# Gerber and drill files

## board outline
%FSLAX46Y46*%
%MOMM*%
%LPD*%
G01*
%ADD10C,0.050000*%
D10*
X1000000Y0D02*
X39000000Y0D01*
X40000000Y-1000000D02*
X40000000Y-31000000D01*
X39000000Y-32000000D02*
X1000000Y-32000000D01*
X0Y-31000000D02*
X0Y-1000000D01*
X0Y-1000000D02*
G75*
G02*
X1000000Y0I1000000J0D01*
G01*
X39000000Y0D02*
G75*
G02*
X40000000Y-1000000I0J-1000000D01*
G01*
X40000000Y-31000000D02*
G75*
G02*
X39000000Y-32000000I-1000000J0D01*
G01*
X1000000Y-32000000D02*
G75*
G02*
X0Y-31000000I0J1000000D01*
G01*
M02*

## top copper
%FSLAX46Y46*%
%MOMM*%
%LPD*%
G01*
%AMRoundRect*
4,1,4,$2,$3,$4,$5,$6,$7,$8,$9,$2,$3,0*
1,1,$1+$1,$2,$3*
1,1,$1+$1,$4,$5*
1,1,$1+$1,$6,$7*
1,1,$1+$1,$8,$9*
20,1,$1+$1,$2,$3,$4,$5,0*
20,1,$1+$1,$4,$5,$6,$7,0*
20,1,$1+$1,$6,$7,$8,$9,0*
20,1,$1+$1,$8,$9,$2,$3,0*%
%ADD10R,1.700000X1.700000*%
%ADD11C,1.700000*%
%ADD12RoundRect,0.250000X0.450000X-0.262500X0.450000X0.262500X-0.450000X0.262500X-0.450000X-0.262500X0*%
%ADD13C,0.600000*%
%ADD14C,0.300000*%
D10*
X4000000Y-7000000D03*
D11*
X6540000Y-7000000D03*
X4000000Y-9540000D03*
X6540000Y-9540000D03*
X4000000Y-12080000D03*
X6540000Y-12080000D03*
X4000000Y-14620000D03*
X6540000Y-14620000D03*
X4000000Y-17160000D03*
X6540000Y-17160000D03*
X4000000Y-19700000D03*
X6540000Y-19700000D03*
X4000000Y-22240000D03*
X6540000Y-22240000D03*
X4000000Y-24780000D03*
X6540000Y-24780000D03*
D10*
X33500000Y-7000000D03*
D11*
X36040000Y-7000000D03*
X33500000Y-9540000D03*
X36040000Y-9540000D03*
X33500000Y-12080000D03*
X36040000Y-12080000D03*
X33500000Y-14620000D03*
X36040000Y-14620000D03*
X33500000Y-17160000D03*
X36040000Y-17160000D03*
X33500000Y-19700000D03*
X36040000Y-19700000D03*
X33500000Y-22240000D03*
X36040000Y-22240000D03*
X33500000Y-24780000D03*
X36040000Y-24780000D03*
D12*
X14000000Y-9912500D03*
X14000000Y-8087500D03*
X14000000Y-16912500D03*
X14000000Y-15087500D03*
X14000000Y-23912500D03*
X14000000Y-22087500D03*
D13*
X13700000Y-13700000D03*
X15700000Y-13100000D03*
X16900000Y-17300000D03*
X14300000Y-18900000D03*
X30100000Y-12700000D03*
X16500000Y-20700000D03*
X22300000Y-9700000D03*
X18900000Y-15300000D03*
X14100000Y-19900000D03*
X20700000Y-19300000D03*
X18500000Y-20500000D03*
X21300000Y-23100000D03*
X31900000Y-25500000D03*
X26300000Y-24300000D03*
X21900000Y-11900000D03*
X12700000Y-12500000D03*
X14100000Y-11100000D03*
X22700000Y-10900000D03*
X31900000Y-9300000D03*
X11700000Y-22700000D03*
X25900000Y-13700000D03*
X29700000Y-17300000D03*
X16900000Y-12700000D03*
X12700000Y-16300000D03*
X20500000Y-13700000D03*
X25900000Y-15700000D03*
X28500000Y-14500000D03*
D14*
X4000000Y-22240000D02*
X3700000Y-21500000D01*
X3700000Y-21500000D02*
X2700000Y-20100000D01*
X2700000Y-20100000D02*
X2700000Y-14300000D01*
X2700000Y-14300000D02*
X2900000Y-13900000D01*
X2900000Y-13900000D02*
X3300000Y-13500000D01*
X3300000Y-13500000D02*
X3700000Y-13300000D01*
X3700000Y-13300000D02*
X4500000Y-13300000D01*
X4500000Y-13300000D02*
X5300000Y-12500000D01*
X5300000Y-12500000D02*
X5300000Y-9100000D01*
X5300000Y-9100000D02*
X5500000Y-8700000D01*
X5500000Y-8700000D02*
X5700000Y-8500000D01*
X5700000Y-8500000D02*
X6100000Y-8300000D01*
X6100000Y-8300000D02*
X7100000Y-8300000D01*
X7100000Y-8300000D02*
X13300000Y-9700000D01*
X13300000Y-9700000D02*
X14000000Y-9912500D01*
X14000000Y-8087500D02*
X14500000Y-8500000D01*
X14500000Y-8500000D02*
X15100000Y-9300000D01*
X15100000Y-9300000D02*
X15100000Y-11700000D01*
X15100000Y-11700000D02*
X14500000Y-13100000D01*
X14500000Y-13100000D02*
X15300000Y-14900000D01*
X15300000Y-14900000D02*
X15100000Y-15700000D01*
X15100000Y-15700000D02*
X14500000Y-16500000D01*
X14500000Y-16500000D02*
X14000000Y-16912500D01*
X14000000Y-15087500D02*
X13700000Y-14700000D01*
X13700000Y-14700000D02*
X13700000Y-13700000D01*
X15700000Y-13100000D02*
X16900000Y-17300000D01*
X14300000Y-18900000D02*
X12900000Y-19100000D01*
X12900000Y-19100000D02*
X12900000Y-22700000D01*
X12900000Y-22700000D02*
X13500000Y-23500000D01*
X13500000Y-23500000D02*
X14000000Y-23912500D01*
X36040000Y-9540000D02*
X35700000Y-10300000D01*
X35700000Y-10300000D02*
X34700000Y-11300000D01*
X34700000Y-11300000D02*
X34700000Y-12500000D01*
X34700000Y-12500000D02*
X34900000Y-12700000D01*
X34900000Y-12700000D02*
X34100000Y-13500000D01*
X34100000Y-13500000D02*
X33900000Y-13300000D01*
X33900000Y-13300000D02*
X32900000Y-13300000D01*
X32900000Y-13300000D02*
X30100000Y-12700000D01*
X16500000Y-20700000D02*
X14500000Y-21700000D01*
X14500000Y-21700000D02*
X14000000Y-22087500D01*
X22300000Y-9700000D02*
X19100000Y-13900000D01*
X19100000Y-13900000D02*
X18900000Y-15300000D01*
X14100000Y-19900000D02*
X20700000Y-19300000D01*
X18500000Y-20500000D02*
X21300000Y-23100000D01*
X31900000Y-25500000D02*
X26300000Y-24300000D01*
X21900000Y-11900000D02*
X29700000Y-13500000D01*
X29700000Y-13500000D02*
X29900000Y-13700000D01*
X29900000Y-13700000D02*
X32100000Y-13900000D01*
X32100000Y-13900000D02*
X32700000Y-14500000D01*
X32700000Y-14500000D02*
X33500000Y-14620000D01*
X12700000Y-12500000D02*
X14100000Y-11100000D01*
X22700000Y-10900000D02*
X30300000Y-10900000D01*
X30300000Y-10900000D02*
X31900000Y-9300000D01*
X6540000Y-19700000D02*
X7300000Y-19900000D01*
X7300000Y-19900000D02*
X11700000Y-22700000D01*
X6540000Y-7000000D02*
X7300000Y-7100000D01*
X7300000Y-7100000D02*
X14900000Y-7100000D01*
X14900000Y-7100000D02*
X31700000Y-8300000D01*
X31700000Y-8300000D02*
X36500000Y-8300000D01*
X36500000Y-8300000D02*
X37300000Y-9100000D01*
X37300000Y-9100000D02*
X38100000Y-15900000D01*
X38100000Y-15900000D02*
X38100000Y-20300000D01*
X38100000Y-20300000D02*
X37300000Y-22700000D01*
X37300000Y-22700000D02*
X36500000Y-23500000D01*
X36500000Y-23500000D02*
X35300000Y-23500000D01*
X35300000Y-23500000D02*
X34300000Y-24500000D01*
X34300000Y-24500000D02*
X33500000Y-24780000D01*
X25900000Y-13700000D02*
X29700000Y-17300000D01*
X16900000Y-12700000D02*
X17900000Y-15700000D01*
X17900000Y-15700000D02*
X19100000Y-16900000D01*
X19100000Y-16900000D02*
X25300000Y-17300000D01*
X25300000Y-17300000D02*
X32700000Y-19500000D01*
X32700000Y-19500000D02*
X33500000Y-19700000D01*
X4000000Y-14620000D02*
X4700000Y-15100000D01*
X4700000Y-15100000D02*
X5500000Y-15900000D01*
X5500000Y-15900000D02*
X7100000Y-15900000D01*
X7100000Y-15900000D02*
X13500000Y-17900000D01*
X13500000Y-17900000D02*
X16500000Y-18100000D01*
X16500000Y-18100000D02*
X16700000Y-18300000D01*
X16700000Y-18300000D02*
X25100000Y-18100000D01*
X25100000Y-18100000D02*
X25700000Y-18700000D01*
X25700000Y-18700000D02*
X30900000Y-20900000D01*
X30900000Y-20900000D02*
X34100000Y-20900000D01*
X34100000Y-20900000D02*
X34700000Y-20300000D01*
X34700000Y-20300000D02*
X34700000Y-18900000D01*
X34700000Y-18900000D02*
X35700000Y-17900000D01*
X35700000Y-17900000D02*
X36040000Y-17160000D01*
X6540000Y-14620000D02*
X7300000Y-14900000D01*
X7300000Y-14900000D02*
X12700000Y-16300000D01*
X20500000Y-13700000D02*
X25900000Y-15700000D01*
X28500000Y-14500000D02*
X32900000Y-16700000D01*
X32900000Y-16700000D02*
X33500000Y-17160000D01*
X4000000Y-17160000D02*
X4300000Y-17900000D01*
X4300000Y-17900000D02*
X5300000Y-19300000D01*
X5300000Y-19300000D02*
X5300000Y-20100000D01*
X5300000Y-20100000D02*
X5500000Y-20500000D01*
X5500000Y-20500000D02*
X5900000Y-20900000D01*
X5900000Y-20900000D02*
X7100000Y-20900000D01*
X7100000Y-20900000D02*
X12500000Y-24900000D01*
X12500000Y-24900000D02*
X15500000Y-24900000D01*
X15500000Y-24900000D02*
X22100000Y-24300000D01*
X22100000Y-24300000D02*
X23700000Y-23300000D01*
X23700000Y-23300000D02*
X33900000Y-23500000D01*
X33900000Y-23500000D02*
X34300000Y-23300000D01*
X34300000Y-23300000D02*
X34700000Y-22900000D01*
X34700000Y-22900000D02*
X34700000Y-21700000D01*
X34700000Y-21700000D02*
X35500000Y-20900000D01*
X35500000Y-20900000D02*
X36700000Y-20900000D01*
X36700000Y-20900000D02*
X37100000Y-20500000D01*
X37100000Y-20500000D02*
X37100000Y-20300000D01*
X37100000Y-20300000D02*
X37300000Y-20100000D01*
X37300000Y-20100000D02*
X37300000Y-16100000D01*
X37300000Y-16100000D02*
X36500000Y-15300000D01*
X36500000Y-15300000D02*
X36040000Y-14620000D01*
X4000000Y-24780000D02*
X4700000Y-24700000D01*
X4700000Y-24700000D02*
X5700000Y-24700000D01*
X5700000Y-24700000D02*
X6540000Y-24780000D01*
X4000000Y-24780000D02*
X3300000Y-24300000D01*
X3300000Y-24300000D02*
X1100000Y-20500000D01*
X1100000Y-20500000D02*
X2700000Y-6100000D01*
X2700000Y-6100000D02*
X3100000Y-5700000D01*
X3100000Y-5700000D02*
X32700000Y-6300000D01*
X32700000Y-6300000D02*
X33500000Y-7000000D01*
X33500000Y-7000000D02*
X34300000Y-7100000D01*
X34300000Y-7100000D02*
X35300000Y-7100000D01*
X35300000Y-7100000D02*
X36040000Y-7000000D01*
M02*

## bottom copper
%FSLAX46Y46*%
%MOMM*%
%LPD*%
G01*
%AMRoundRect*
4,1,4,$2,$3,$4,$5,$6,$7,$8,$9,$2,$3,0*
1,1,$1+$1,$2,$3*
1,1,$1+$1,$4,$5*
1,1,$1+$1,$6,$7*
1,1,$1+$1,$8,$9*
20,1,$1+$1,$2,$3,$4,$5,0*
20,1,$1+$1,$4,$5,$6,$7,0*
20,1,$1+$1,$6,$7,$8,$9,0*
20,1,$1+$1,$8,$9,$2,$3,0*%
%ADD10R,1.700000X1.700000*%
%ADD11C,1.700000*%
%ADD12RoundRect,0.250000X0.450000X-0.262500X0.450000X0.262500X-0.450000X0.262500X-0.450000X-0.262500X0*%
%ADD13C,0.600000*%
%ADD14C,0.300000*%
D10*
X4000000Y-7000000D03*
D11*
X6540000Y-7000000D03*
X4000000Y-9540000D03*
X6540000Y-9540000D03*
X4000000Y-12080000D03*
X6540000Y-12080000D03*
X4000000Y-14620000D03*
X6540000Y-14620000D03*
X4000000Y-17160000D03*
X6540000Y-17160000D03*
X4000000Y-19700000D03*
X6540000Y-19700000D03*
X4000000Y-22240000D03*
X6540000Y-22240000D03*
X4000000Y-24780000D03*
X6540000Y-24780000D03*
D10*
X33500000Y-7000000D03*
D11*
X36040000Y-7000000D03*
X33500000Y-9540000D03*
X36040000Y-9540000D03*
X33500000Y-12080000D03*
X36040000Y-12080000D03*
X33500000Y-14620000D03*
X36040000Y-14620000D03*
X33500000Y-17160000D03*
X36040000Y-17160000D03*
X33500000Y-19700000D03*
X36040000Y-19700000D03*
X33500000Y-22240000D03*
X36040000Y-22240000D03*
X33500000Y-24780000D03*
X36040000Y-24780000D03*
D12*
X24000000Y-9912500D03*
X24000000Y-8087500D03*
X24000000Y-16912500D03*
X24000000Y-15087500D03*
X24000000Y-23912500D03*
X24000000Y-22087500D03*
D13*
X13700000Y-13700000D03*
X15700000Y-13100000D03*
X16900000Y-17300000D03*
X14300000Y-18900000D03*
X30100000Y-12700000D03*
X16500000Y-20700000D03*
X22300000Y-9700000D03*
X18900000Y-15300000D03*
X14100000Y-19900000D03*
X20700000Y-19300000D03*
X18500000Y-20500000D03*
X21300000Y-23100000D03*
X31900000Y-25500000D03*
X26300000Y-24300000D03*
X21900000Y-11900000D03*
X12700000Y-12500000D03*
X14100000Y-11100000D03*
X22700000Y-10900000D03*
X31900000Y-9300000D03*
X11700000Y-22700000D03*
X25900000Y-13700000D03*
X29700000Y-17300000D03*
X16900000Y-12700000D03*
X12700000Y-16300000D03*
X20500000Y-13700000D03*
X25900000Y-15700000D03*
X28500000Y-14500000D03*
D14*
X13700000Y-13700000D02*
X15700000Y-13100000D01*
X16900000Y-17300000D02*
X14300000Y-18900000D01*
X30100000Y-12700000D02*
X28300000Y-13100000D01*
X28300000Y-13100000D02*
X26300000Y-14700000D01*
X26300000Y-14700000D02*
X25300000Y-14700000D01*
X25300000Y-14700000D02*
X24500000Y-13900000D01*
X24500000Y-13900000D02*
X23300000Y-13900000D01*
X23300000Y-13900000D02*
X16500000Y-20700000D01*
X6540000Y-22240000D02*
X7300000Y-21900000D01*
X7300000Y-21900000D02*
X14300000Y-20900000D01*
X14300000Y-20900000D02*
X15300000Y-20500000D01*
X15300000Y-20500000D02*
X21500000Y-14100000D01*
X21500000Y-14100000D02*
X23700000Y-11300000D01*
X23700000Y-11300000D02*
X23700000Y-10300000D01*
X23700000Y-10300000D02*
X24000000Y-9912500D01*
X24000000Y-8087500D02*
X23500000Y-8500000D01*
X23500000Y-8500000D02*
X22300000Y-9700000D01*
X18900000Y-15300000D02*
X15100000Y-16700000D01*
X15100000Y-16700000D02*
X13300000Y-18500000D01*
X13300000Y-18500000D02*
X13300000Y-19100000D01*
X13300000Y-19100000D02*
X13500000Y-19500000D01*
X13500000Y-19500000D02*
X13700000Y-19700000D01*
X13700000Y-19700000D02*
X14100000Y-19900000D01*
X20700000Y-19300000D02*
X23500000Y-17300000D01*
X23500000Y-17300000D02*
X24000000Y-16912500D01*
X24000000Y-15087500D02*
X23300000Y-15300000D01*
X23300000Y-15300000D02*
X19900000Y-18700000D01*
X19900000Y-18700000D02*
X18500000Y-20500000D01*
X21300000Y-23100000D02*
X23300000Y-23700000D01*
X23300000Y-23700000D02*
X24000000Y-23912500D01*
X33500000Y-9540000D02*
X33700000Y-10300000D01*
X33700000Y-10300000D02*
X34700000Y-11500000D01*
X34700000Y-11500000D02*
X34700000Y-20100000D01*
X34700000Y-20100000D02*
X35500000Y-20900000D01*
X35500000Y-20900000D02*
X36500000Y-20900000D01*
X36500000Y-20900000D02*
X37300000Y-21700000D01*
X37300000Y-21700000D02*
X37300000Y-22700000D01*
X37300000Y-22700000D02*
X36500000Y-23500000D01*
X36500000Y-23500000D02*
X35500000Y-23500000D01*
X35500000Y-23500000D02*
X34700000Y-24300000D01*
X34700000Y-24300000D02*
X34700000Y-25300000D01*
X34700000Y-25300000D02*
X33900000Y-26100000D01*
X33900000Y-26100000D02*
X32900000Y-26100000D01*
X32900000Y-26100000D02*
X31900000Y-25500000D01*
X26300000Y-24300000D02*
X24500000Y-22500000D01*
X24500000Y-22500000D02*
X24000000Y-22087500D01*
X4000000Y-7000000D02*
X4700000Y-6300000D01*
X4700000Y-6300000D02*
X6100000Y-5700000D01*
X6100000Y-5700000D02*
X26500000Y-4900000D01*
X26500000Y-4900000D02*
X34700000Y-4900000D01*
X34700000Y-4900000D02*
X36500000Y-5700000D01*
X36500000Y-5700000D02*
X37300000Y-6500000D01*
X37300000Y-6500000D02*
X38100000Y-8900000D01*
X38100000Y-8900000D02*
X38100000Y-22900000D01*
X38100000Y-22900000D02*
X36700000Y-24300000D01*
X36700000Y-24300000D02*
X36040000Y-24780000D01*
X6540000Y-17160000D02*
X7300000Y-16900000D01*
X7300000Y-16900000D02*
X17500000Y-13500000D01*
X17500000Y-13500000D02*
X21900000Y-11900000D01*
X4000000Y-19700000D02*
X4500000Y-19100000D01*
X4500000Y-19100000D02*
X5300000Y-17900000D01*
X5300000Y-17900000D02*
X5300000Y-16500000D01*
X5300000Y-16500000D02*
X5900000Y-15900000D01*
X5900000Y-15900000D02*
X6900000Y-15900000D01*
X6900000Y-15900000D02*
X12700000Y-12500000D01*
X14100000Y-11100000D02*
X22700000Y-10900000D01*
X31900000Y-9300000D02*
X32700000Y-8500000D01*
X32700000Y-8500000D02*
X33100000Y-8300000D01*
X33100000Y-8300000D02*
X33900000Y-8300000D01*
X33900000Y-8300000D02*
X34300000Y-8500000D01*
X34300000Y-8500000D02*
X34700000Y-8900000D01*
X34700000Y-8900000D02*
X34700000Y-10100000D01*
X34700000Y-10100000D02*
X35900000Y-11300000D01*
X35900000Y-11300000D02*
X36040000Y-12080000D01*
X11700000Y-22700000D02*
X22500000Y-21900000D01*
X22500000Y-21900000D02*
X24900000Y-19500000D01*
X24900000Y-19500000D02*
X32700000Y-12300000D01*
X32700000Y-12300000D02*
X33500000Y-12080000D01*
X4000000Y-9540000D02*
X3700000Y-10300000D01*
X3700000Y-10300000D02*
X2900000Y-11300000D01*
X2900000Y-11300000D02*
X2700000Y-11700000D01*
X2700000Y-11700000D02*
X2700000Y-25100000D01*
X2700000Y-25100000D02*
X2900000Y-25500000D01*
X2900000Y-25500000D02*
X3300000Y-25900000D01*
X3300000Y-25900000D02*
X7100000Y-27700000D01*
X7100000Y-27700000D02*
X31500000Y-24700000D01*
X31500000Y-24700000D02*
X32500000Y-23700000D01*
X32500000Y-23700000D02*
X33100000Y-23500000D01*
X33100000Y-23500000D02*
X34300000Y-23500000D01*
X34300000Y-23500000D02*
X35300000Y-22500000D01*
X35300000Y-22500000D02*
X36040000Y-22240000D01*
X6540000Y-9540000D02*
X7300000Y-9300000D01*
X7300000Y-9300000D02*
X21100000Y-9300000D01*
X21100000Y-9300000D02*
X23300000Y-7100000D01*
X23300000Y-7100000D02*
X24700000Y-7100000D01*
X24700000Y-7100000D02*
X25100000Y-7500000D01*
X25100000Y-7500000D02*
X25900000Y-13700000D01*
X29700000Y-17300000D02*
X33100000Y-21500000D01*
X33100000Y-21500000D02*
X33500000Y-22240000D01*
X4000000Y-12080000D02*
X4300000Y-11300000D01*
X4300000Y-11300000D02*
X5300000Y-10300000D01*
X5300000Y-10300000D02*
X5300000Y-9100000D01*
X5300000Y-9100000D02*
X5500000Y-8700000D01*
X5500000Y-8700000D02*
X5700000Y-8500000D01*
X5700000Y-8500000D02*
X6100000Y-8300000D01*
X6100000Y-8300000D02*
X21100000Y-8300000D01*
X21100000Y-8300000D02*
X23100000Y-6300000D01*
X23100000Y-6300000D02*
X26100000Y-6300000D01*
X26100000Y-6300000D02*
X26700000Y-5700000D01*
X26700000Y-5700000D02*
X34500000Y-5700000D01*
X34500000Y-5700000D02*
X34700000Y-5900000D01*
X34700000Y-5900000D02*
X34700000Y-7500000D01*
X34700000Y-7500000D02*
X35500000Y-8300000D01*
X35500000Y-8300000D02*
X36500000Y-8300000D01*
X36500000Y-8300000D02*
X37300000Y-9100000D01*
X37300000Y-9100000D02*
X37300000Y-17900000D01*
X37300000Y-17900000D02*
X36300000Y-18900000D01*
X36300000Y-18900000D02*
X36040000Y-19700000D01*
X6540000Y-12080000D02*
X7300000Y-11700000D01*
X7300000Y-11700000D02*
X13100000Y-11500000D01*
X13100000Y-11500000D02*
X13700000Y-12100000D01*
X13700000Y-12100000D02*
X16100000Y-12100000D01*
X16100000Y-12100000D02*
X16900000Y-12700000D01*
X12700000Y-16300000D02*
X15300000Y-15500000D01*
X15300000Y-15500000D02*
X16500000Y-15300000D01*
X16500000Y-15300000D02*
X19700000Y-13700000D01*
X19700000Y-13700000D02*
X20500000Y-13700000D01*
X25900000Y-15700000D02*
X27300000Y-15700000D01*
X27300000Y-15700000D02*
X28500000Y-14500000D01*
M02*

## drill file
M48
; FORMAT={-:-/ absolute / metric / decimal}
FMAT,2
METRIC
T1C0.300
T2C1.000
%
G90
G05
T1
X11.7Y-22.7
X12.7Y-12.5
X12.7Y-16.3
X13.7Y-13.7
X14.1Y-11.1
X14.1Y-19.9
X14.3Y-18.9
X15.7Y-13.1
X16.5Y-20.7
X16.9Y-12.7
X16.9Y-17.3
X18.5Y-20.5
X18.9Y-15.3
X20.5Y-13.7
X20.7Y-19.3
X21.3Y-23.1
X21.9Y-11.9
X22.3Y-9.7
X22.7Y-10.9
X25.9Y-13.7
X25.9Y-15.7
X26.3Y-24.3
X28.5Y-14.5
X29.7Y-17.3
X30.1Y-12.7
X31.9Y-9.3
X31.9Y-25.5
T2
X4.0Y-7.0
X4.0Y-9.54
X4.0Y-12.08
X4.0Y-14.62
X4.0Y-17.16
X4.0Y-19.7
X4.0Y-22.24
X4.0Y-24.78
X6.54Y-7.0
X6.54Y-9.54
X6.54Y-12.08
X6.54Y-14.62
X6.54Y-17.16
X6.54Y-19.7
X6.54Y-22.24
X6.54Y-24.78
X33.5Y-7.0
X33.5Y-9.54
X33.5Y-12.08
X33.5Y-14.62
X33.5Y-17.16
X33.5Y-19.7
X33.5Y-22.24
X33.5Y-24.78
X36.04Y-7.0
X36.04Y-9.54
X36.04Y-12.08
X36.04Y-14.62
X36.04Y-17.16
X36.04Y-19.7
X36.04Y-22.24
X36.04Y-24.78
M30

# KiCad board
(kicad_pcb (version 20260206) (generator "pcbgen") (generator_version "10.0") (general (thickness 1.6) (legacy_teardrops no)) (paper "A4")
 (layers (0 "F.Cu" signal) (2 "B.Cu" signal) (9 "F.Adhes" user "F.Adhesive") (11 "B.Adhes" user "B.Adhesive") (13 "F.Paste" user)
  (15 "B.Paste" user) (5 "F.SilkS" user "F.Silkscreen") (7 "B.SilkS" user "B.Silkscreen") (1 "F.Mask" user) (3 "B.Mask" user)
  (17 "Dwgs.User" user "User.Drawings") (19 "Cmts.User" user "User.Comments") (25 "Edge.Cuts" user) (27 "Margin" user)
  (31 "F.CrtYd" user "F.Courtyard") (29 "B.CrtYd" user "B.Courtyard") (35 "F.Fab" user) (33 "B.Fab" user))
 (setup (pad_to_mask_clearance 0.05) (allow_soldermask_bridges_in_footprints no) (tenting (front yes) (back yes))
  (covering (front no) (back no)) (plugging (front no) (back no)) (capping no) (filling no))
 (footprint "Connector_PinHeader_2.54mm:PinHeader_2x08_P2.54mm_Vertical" (layer "F.Cu") (at 4 7)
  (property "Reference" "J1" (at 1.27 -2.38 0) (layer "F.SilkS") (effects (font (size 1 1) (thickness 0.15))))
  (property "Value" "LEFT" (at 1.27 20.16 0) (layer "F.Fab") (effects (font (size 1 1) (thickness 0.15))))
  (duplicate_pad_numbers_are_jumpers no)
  (pad "1" thru_hole rect (at 0 0) (size 1.7 1.7) (drill 1) (layers "*.Cu" "*.Mask") (remove_unused_layers no) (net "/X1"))
  (pad "2" thru_hole circle (at 2.54 0) (size 1.7 1.7) (drill 1) (layers "*.Cu" "*.Mask") (remove_unused_layers no) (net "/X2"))
  (pad "3" thru_hole circle (at 0 2.54) (size 1.7 1.7) (drill 1) (layers "*.Cu" "*.Mask") (remove_unused_layers no) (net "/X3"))
  (pad "4" thru_hole circle (at 2.54 2.54) (size 1.7 1.7) (drill 1) (layers "*.Cu" "*.Mask") (remove_unused_layers no) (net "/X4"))
  (pad "5" thru_hole circle (at 0 5.08) (size 1.7 1.7) (drill 1) (layers "*.Cu" "*.Mask") (remove_unused_layers no) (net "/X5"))
  (pad "6" thru_hole circle (at 2.54 5.08) (size 1.7 1.7) (drill 1) (layers "*.Cu" "*.Mask") (remove_unused_layers no) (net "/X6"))
  (pad "7" thru_hole circle (at 0 7.62) (size 1.7 1.7) (drill 1) (layers "*.Cu" "*.Mask") (remove_unused_layers no) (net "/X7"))
  (pad "8" thru_hole circle (at 2.54 7.62) (size 1.7 1.7) (drill 1) (layers "*.Cu" "*.Mask") (remove_unused_layers no) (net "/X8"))
  (pad "9" thru_hole circle (at 0 10.16) (size 1.7 1.7) (drill 1) (layers "*.Cu" "*.Mask") (remove_unused_layers no) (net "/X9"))
  (pad "10" thru_hole circle (at 2.54 10.16) (size 1.7 1.7) (drill 1) (layers "*.Cu" "*.Mask") (remove_unused_layers no) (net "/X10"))
  (pad "11" thru_hole circle (at 0 12.7) (size 1.7 1.7) (drill 1) (layers "*.Cu" "*.Mask") (remove_unused_layers no) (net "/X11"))
  (pad "12" thru_hole circle (at 2.54 12.7) (size 1.7 1.7) (drill 1) (layers "*.Cu" "*.Mask") (remove_unused_layers no) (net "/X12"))
  (pad "13" thru_hole circle (at 0 15.24) (size 1.7 1.7) (drill 1) (layers "*.Cu" "*.Mask") (remove_unused_layers no) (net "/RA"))
  (pad "14" thru_hole circle (at 2.54 15.24) (size 1.7 1.7) (drill 1) (layers "*.Cu" "*.Mask") (remove_unused_layers no) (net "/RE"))
  (pad "15" thru_hole circle (at 0 17.78) (size 1.7 1.7) (drill 1) (layers "*.Cu" "*.Mask") (remove_unused_layers no) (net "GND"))
  (pad "16" thru_hole circle (at 2.54 17.78) (size 1.7 1.7) (drill 1) (layers "*.Cu" "*.Mask") (remove_unused_layers no) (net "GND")))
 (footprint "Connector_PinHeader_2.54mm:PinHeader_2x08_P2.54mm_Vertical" (layer "F.Cu") (at 33.5 7)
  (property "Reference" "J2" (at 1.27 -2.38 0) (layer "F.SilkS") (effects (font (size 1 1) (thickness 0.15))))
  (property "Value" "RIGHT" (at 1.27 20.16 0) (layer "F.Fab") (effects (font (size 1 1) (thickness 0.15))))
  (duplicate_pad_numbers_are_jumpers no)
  (pad "1" thru_hole rect (at 0 0) (size 1.7 1.7) (drill 1) (layers "*.Cu" "*.Mask") (remove_unused_layers no) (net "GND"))
  (pad "2" thru_hole circle (at 2.54 0) (size 1.7 1.7) (drill 1) (layers "*.Cu" "*.Mask") (remove_unused_layers no) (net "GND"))
  (pad "3" thru_hole circle (at 0 2.54) (size 1.7 1.7) (drill 1) (layers "*.Cu" "*.Mask") (remove_unused_layers no) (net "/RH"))
  (pad "4" thru_hole circle (at 2.54 2.54) (size 1.7 1.7) (drill 1) (layers "*.Cu" "*.Mask") (remove_unused_layers no) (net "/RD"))
  (pad "5" thru_hole circle (at 0 5.08) (size 1.7 1.7) (drill 1) (layers "*.Cu" "*.Mask") (remove_unused_layers no) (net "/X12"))
  (pad "6" thru_hole circle (at 2.54 5.08) (size 1.7 1.7) (drill 1) (layers "*.Cu" "*.Mask") (remove_unused_layers no) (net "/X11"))
  (pad "7" thru_hole circle (at 0 7.62) (size 1.7 1.7) (drill 1) (layers "*.Cu" "*.Mask") (remove_unused_layers no) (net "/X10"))
  (pad "8" thru_hole circle (at 2.54 7.62) (size 1.7 1.7) (drill 1) (layers "*.Cu" "*.Mask") (remove_unused_layers no) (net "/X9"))
  (pad "9" thru_hole circle (at 0 10.16) (size 1.7 1.7) (drill 1) (layers "*.Cu" "*.Mask") (remove_unused_layers no) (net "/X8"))
  (pad "10" thru_hole circle (at 2.54 10.16) (size 1.7 1.7) (drill 1) (layers "*.Cu" "*.Mask") (remove_unused_layers no) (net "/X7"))
  (pad "11" thru_hole circle (at 0 12.7) (size 1.7 1.7) (drill 1) (layers "*.Cu" "*.Mask") (remove_unused_layers no) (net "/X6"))
  (pad "12" thru_hole circle (at 2.54 12.7) (size 1.7 1.7) (drill 1) (layers "*.Cu" "*.Mask") (remove_unused_layers no) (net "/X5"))
  (pad "13" thru_hole circle (at 0 15.24) (size 1.7 1.7) (drill 1) (layers "*.Cu" "*.Mask") (remove_unused_layers no) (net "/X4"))
  (pad "14" thru_hole circle (at 2.54 15.24) (size 1.7 1.7) (drill 1) (layers "*.Cu" "*.Mask") (remove_unused_layers no) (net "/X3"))
  (pad "15" thru_hole circle (at 0 17.78) (size 1.7 1.7) (drill 1) (layers "*.Cu" "*.Mask") (remove_unused_layers no) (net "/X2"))
  (pad "16" thru_hole circle (at 2.54 17.78) (size 1.7 1.7) (drill 1) (layers "*.Cu" "*.Mask") (remove_unused_layers no) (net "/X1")))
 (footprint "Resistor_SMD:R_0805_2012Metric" (layer "F.Cu") (at 14 9 90)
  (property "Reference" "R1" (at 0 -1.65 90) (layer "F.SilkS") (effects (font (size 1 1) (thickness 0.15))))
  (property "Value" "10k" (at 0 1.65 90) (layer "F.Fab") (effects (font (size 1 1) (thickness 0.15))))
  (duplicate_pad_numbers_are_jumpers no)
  (pad "1" smd roundrect (at -0.9125 0 90) (size 1.025 1.4) (layers "F.Cu" "F.Mask" "F.Paste") (roundrect_rratio 0.243902) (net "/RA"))
  (pad "2" smd roundrect (at 0.9125 0 90) (size 1.025 1.4) (layers "F.Cu" "F.Mask" "F.Paste") (roundrect_rratio 0.243902) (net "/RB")))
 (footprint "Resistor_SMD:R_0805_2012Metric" (layer "F.Cu") (at 14 16 90)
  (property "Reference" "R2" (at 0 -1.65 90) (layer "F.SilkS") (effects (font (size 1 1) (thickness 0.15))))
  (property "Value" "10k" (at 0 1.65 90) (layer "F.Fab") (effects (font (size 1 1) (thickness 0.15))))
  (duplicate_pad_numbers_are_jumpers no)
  (pad "1" smd roundrect (at -0.9125 0 90) (size 1.025 1.4) (layers "F.Cu" "F.Mask" "F.Paste") (roundrect_rratio 0.243902) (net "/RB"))
  (pad "2" smd roundrect (at 0.9125 0 90) (size 1.025 1.4) (layers "F.Cu" "F.Mask" "F.Paste") (roundrect_rratio 0.243902) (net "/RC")))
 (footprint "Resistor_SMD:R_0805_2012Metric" (layer "F.Cu") (at 14 23 90)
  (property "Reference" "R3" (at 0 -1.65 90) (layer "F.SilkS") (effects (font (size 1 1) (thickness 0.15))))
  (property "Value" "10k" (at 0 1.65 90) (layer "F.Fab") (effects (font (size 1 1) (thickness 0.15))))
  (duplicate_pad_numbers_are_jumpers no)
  (pad "1" smd roundrect (at -0.9125 0 90) (size 1.025 1.4) (layers "F.Cu" "F.Mask" "F.Paste") (roundrect_rratio 0.243902) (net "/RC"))
  (pad "2" smd roundrect (at 0.9125 0 90) (size 1.025 1.4) (layers "F.Cu" "F.Mask" "F.Paste") (roundrect_rratio 0.243902) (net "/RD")))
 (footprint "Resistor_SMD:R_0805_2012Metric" (layer "B.Cu") (at 24 9 90)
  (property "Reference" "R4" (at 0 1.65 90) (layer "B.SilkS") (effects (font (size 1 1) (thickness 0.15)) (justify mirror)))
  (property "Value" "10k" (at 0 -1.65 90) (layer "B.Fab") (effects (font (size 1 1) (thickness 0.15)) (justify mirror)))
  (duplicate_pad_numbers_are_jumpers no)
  (pad "1" smd roundrect (at -0.9125 0 90) (size 1.025 1.4) (layers "B.Cu" "B.Mask" "B.Paste") (roundrect_rratio 0.243902) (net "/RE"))
  (pad "2" smd roundrect (at 0.9125 0 90) (size 1.025 1.4) (layers "B.Cu" "B.Mask" "B.Paste") (roundrect_rratio 0.243902) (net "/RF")))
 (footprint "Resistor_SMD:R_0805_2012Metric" (layer "B.Cu") (at 24 16 90)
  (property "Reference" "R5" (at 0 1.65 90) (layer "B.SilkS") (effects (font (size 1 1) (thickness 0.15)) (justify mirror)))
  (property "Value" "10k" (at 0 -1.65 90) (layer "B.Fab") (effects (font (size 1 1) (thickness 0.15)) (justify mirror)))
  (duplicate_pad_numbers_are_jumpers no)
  (pad "1" smd roundrect (at -0.9125 0 90) (size 1.025 1.4) (layers "B.Cu" "B.Mask" "B.Paste") (roundrect_rratio 0.243902) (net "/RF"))
  (pad "2" smd roundrect (at 0.9125 0 90) (size 1.025 1.4) (layers "B.Cu" "B.Mask" "B.Paste") (roundrect_rratio 0.243902) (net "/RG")))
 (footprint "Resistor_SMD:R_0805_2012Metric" (layer "B.Cu") (at 24 23 90)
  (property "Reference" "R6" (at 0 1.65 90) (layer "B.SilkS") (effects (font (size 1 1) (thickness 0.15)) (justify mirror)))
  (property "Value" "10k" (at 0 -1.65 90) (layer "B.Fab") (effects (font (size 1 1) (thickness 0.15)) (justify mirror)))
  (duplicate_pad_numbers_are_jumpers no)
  (pad "1" smd roundrect (at -0.9125 0 90) (size 1.025 1.4) (layers "B.Cu" "B.Mask" "B.Paste") (roundrect_rratio 0.243902) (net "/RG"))
  (pad "2" smd roundrect (at 0.9125 0 90) (size 1.025 1.4) (layers "B.Cu" "B.Mask" "B.Paste") (roundrect_rratio 0.243902) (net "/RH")))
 (gr_line (start 1 0) (end 39 0) (stroke (width 0.05) (type default)) (layer "Edge.Cuts"))
 (gr_line (start 40 1) (end 40 31) (stroke (width 0.05) (type default)) (layer "Edge.Cuts"))
 (gr_line (start 39 32) (end 1 32) (stroke (width 0.05) (type default)) (layer "Edge.Cuts"))
 (gr_line (start 0 31) (end 0 1) (stroke (width 0.05) (type default)) (layer "Edge.Cuts"))
 (gr_arc (start 0 1) (mid 0.292893 0.292893) (end 1 0) (stroke (width 0.05) (type default)) (layer "Edge.Cuts"))
 (gr_arc (start 39 0) (mid 39.707107 0.292893) (end 40 1) (stroke (width 0.05) (type default)) (layer "Edge.Cuts"))
 (gr_arc (start 40 31) (mid 39.707107 31.707107) (end 39 32) (stroke (width 0.05) (type default)) (layer "Edge.Cuts"))
 (gr_arc (start 1 32) (mid 0.292893 31.707107) (end 0 31) (stroke (width 0.05) (type default)) (layer "Edge.Cuts"))
 (segment (start 4 22.24) (end 3.7 21.5) (width 0.3) (layer "F.Cu") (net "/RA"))
 (segment (start 3.7 21.5) (end 2.7 20.1) (width 0.3) (layer "F.Cu") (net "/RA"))
 (segment (start 2.7 20.1) (end 2.7 14.3) (width 0.3) (layer "F.Cu") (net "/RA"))
 (segment (start 2.7 14.3) (end 2.9 13.9) (width 0.3) (layer "F.Cu") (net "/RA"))
 (segment (start 2.9 13.9) (end 3.3 13.5) (width 0.3) (layer "F.Cu") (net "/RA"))
 (segment (start 3.3 13.5) (end 3.7 13.3) (width 0.3) (layer "F.Cu") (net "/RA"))
 (segment (start 3.7 13.3) (end 4.5 13.3) (width 0.3) (layer "F.Cu") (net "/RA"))
 (segment (start 4.5 13.3) (end 5.3 12.5) (width 0.3) (layer "F.Cu") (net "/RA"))
 (segment (start 5.3 12.5) (end 5.3 9.1) (width 0.3) (layer "F.Cu") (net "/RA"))
 (segment (start 5.3 9.1) (end 5.5 8.7) (width 0.3) (layer "F.Cu") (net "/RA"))
 (segment (start 5.5 8.7) (end 5.7 8.5) (width 0.3) (layer "F.Cu") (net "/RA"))
 (segment (start 5.7 8.5) (end 6.1 8.3) (width 0.3) (layer "F.Cu") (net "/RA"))
 (segment (start 6.1 8.3) (end 7.1 8.3) (width 0.3) (layer "F.Cu") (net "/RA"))
 (segment (start 7.1 8.3) (end 13.3 9.7) (width 0.3) (layer "F.Cu") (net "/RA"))
 (segment (start 13.3 9.7) (end 14 9.9125) (width 0.3) (layer "F.Cu") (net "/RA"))
 (segment (start 14 8.0875) (end 14.5 8.5) (width 0.3) (layer "F.Cu") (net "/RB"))
 (segment (start 14.5 8.5) (end 15.1 9.3) (width 0.3) (layer "F.Cu") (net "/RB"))
 (segment (start 15.1 9.3) (end 15.1 11.7) (width 0.3) (layer "F.Cu") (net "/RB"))
 (segment (start 15.1 11.7) (end 14.5 13.1) (width 0.3) (layer "F.Cu") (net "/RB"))
 (segment (start 14.5 13.1) (end 15.3 14.9) (width 0.3) (layer "F.Cu") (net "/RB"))
 (segment (start 15.3 14.9) (end 15.1 15.7) (width 0.3) (layer "F.Cu") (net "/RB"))
 (segment (start 15.1 15.7) (end 14.5 16.5) (width 0.3) (layer "F.Cu") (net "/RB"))
 (segment (start 14.5 16.5) (end 14 16.9125) (width 0.3) (layer "F.Cu") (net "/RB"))
 (segment (start 14 15.0875) (end 13.7 14.7) (width 0.3) (layer "F.Cu") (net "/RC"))
 (segment (start 13.7 14.7) (end 13.7 13.7) (width 0.3) (layer "F.Cu") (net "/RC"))
 (segment (start 13.7 13.7) (end 15.7 13.1) (width 0.3) (layer "B.Cu") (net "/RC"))
 (segment (start 15.7 13.1) (end 16.9 17.3) (width 0.3) (layer "F.Cu") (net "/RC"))
 (segment (start 16.9 17.3) (end 14.3 18.9) (width 0.3) (layer "B.Cu") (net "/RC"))
 (segment (start 14.3 18.9) (end 12.9 19.1) (width 0.3) (layer "F.Cu") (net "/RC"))
 (segment (start 12.9 19.1) (end 12.9 22.7) (width 0.3) (layer "F.Cu") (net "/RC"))
 (segment (start 12.9 22.7) (end 13.5 23.5) (width 0.3) (layer "F.Cu") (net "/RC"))
 (segment (start 13.5 23.5) (end 14 23.9125) (width 0.3) (layer "F.Cu") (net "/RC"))
 (segment (start 36.04 9.54) (end 35.7 10.3) (width 0.3) (layer "F.Cu") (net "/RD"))
 (segment (start 35.7 10.3) (end 34.7 11.3) (width 0.3) (layer "F.Cu") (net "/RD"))
 (segment (start 34.7 11.3) (end 34.7 12.5) (width 0.3) (layer "F.Cu") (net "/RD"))
 (segment (start 34.7 12.5) (end 34.9 12.7) (width 0.3) (layer "F.Cu") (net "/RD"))
 (segment (start 34.9 12.7) (end 34.1 13.5) (width 0.3) (layer "F.Cu") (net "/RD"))
 (segment (start 34.1 13.5) (end 33.9 13.3) (width 0.3) (layer "F.Cu") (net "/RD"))
 (segment (start 33.9 13.3) (end 32.9 13.3) (width 0.3) (layer "F.Cu") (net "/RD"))
 (segment (start 32.9 13.3) (end 30.1 12.7) (width 0.3) (layer "F.Cu") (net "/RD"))
 (segment (start 30.1 12.7) (end 28.3 13.1) (width 0.3) (layer "B.Cu") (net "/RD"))
 (segment (start 28.3 13.1) (end 26.3 14.7) (width 0.3) (layer "B.Cu") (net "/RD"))
 (segment (start 26.3 14.7) (end 25.3 14.7) (width 0.3) (layer "B.Cu") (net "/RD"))
 (segment (start 25.3 14.7) (end 24.5 13.9) (width 0.3) (layer "B.Cu") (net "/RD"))
 (segment (start 24.5 13.9) (end 23.3 13.9) (width 0.3) (layer "B.Cu") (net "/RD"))
 (segment (start 23.3 13.9) (end 16.5 20.7) (width 0.3) (layer "B.Cu") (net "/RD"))
 (segment (start 16.5 20.7) (end 14.5 21.7) (width 0.3) (layer "F.Cu") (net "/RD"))
 (segment (start 14.5 21.7) (end 14 22.0875) (width 0.3) (layer "F.Cu") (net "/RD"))
 (segment (start 6.54 22.24) (end 7.3 21.9) (width 0.3) (layer "B.Cu") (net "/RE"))
 (segment (start 7.3 21.9) (end 14.3 20.9) (width 0.3) (layer "B.Cu") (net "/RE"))
 (segment (start 14.3 20.9) (end 15.3 20.5) (width 0.3) (layer "B.Cu") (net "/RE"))
 (segment (start 15.3 20.5) (end 21.5 14.1) (width 0.3) (layer "B.Cu") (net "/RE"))
 (segment (start 21.5 14.1) (end 23.7 11.3) (width 0.3) (layer "B.Cu") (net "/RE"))
 (segment (start 23.7 11.3) (end 23.7 10.3) (width 0.3) (layer "B.Cu") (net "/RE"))
 (segment (start 23.7 10.3) (end 24 9.9125) (width 0.3) (layer "B.Cu") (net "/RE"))
 (segment (start 24 8.0875) (end 23.5 8.5) (width 0.3) (layer "B.Cu") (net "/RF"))
 (segment (start 23.5 8.5) (end 22.3 9.7) (width 0.3) (layer "B.Cu") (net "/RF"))
 (segment (start 22.3 9.7) (end 19.1 13.9) (width 0.3) (layer "F.Cu") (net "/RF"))
 (segment (start 19.1 13.9) (end 18.9 15.3) (width 0.3) (layer "F.Cu") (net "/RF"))
 (segment (start 18.9 15.3) (end 15.1 16.7) (width 0.3) (layer "B.Cu") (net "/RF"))
 (segment (start 15.1 16.7) (end 13.3 18.5) (width 0.3) (layer "B.Cu") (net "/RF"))
 (segment (start 13.3 18.5) (end 13.3 19.1) (width 0.3) (layer "B.Cu") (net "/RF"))
 (segment (start 13.3 19.1) (end 13.5 19.5) (width 0.3) (layer "B.Cu") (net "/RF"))
 (segment (start 13.5 19.5) (end 13.7 19.7) (width 0.3) (layer "B.Cu") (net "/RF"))
 (segment (start 13.7 19.7) (end 14.1 19.9) (width 0.3) (layer "B.Cu") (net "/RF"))
 (segment (start 14.1 19.9) (end 20.7 19.3) (width 0.3) (layer "F.Cu") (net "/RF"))
 (segment (start 20.7 19.3) (end 23.5 17.3) (width 0.3) (layer "B.Cu") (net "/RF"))
 (segment (start 23.5 17.3) (end 24 16.9125) (width 0.3) (layer "B.Cu") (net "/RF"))
 (segment (start 24 15.0875) (end 23.3 15.3) (width 0.3) (layer "B.Cu") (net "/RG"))
 (segment (start 23.3 15.3) (end 19.9 18.7) (width 0.3) (layer "B.Cu") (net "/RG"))
 (segment (start 19.9 18.7) (end 18.5 20.5) (width 0.3) (layer "B.Cu") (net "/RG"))
 (segment (start 18.5 20.5) (end 21.3 23.1) (width 0.3) (layer "F.Cu") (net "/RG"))
 (segment (start 21.3 23.1) (end 23.3 23.7) (width 0.3) (layer "B.Cu") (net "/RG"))
 (segment (start 23.3 23.7) (end 24 23.9125) (width 0.3) (layer "B.Cu") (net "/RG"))
 (segment (start 33.5 9.54) (end 33.7 10.3) (width 0.3) (layer "B.Cu") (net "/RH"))
 (segment (start 33.7 10.3) (end 34.7 11.5) (width 0.3) (layer "B.Cu") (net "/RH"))
 (segment (start 34.7 11.5) (end 34.7 20.1) (width 0.3) (layer "B.Cu") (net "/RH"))
 (segment (start 34.7 20.1) (end 35.5 20.9) (width 0.3) (layer "B.Cu") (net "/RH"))
 (segment (start 35.5 20.9) (end 36.5 20.9) (width 0.3) (layer "B.Cu") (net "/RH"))
 (segment (start 36.5 20.9) (end 37.3 21.7) (width 0.3) (layer "B.Cu") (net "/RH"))
 (segment (start 37.3 21.7) (end 37.3 22.7) (width 0.3) (layer "B.Cu") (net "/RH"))
 (segment (start 37.3 22.7) (end 36.5 23.5) (width 0.3) (layer "B.Cu") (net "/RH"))
 (segment (start 36.5 23.5) (end 35.5 23.5) (width 0.3) (layer "B.Cu") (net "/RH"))
 (segment (start 35.5 23.5) (end 34.7 24.3) (width 0.3) (layer "B.Cu") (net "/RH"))
 (segment (start 34.7 24.3) (end 34.7 25.3) (width 0.3) (layer "B.Cu") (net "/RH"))
 (segment (start 34.7 25.3) (end 33.9 26.1) (width 0.3) (layer "B.Cu") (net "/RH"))
 (segment (start 33.9 26.1) (end 32.9 26.1) (width 0.3) (layer "B.Cu") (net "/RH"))
 (segment (start 32.9 26.1) (end 31.9 25.5) (width 0.3) (layer "B.Cu") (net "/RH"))
 (segment (start 31.9 25.5) (end 26.3 24.3) (width 0.3) (layer "F.Cu") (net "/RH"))
 (segment (start 26.3 24.3) (end 24.5 22.5) (width 0.3) (layer "B.Cu") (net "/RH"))
 (segment (start 24.5 22.5) (end 24 22.0875) (width 0.3) (layer "B.Cu") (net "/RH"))
 (segment (start 4 7) (end 4.7 6.3) (width 0.3) (layer "B.Cu") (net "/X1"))
 (segment (start 4.7 6.3) (end 6.1 5.7) (width 0.3) (layer "B.Cu") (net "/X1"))
 (segment (start 6.1 5.7) (end 26.5 4.9) (width 0.3) (layer "B.Cu") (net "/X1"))
 (segment (start 26.5 4.9) (end 34.7 4.9) (width 0.3) (layer "B.Cu") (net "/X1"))
 (segment (start 34.7 4.9) (end 36.5 5.7) (width 0.3) (layer "B.Cu") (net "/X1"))
 (segment (start 36.5 5.7) (end 37.3 6.5) (width 0.3) (layer "B.Cu") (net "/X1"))
 (segment (start 37.3 6.5) (end 38.1 8.9) (width 0.3) (layer "B.Cu") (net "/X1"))
 (segment (start 38.1 8.9) (end 38.1 22.9) (width 0.3) (layer "B.Cu") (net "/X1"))
 (segment (start 38.1 22.9) (end 36.7 24.3) (width 0.3) (layer "B.Cu") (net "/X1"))
 (segment (start 36.7 24.3) (end 36.04 24.78) (width 0.3) (layer "B.Cu") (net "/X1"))
 (segment (start 6.54 17.16) (end 7.3 16.9) (width 0.3) (layer "B.Cu") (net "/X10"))
 (segment (start 7.3 16.9) (end 17.5 13.5) (width 0.3) (layer "B.Cu") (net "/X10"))
 (segment (start 17.5 13.5) (end 21.9 11.9) (width 0.3) (layer "B.Cu") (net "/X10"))
 (segment (start 21.9 11.9) (end 29.7 13.5) (width 0.3) (layer "F.Cu") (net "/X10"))
 (segment (start 29.7 13.5) (end 29.9 13.7) (width 0.3) (layer "F.Cu") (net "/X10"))
 (segment (start 29.9 13.7) (end 32.1 13.9) (width 0.3) (layer "F.Cu") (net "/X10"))
 (segment (start 32.1 13.9) (end 32.7 14.5) (width 0.3) (layer "F.Cu") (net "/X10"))
 (segment (start 32.7 14.5) (end 33.5 14.62) (width 0.3) (layer "F.Cu") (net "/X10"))
 (segment (start 4 19.7) (end 4.5 19.1) (width 0.3) (layer "B.Cu") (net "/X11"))
 (segment (start 4.5 19.1) (end 5.3 17.9) (width 0.3) (layer "B.Cu") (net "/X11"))
 (segment (start 5.3 17.9) (end 5.3 16.5) (width 0.3) (layer "B.Cu") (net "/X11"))
 (segment (start 5.3 16.5) (end 5.9 15.9) (width 0.3) (layer "B.Cu") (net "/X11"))
 (segment (start 5.9 15.9) (end 6.9 15.9) (width 0.3) (layer "B.Cu") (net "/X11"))
 (segment (start 6.9 15.9) (end 12.7 12.5) (width 0.3) (layer "B.Cu") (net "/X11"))
 (segment (start 12.7 12.5) (end 14.1 11.1) (width 0.3) (layer "F.Cu") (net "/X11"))
 (segment (start 14.1 11.1) (end 22.7 10.9) (width 0.3) (layer "B.Cu") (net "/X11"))
 (segment (start 22.7 10.9) (end 30.3 10.9) (width 0.3) (layer "F.Cu") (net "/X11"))
 (segment (start 30.3 10.9) (end 31.9 9.3) (width 0.3) (layer "F.Cu") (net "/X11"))
 (segment (start 31.9 9.3) (end 32.7 8.5) (width 0.3) (layer "B.Cu") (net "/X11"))
 (segment (start 32.7 8.5) (end 33.1 8.3) (width 0.3) (layer "B.Cu") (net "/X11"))
 (segment (start 33.1 8.3) (end 33.9 8.3) (width 0.3) (layer "B.Cu") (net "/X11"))
 (segment (start 33.9 8.3) (end 34.3 8.5) (width 0.3) (layer "B.Cu") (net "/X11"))
 (segment (start 34.3 8.5) (end 34.7 8.9) (width 0.3) (layer "B.Cu") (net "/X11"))
 (segment (start 34.7 8.9) (end 34.7 10.1) (width 0.3) (layer "B.Cu") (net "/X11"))
 (segment (start 34.7 10.1) (end 35.9 11.3) (width 0.3) (layer "B.Cu") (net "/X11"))
 (segment (start 35.9 11.3) (end 36.04 12.08) (width 0.3) (layer "B.Cu") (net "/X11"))
 (segment (start 6.54 19.7) (end 7.3 19.9) (width 0.3) (layer "F.Cu") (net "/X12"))
 (segment (start 7.3 19.9) (end 11.7 22.7) (width 0.3) (layer "F.Cu") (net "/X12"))
 (segment (start 11.7 22.7) (end 22.5 21.9) (width 0.3) (layer "B.Cu") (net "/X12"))
 (segment (start 22.5 21.9) (end 24.9 19.5) (width 0.3) (layer "B.Cu") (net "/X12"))
 (segment (start 24.9 19.5) (end 32.7 12.3) (width 0.3) (layer "B.Cu") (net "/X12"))
 (segment (start 32.7 12.3) (end 33.5 12.08) (width 0.3) (layer "B.Cu") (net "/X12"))
 (segment (start 6.54 7) (end 7.3 7.1) (width 0.3) (layer "F.Cu") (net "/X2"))
 (segment (start 7.3 7.1) (end 14.9 7.1) (width 0.3) (layer "F.Cu") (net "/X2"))
 (segment (start 14.9 7.1) (end 31.7 8.3) (width 0.3) (layer "F.Cu") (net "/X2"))
 (segment (start 31.7 8.3) (end 36.5 8.3) (width 0.3) (layer "F.Cu") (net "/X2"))
 (segment (start 36.5 8.3) (end 37.3 9.1) (width 0.3) (layer "F.Cu") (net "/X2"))
 (segment (start 37.3 9.1) (end 38.1 15.9) (width 0.3) (layer "F.Cu") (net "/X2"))
 (segment (start 38.1 15.9) (end 38.1 20.3) (width 0.3) (layer "F.Cu") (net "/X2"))
 (segment (start 38.1 20.3) (end 37.3 22.7) (width 0.3) (layer "F.Cu") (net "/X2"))
 (segment (start 37.3 22.7) (end 36.5 23.5) (width 0.3) (layer "F.Cu") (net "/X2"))
 (segment (start 36.5 23.5) (end 35.3 23.5) (width 0.3) (layer "F.Cu") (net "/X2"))
 (segment (start 35.3 23.5) (end 34.3 24.5) (width 0.3) (layer "F.Cu") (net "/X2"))
 (segment (start 34.3 24.5) (end 33.5 24.78) (width 0.3) (layer "F.Cu") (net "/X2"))
 (segment (start 4 9.54) (end 3.7 10.3) (width 0.3) (layer "B.Cu") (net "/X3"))
 (segment (start 3.7 10.3) (end 2.9 11.3) (width 0.3) (layer "B.Cu") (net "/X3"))
 (segment (start 2.9 11.3) (end 2.7 11.7) (width 0.3) (layer "B.Cu") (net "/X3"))
 (segment (start 2.7 11.7) (end 2.7 25.1) (width 0.3) (layer "B.Cu") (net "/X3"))
 (segment (start 2.7 25.1) (end 2.9 25.5) (width 0.3) (layer "B.Cu") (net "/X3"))
 (segment (start 2.9 25.5) (end 3.3 25.9) (width 0.3) (layer "B.Cu") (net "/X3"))
 (segment (start 3.3 25.9) (end 7.1 27.7) (width 0.3) (layer "B.Cu") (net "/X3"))
 (segment (start 7.1 27.7) (end 31.5 24.7) (width 0.3) (layer "B.Cu") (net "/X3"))
 (segment (start 31.5 24.7) (end 32.5 23.7) (width 0.3) (layer "B.Cu") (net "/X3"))
 (segment (start 32.5 23.7) (end 33.1 23.5) (width 0.3) (layer "B.Cu") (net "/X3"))
 (segment (start 33.1 23.5) (end 34.3 23.5) (width 0.3) (layer "B.Cu") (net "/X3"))
 (segment (start 34.3 23.5) (end 35.3 22.5) (width 0.3) (layer "B.Cu") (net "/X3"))
 (segment (start 35.3 22.5) (end 36.04 22.24) (width 0.3) (layer "B.Cu") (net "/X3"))
 (segment (start 6.54 9.54) (end 7.3 9.3) (width 0.3) (layer "B.Cu") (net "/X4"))
 (segment (start 7.3 9.3) (end 21.1 9.3) (width 0.3) (layer "B.Cu") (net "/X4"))
 (segment (start 21.1 9.3) (end 23.3 7.1) (width 0.3) (layer "B.Cu") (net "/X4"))
 (segment (start 23.3 7.1) (end 24.7 7.1) (width 0.3) (layer "B.Cu") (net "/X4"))
 (segment (start 24.7 7.1) (end 25.1 7.5) (width 0.3) (layer "B.Cu") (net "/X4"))
 (segment (start 25.1 7.5) (end 25.9 13.7) (width 0.3) (layer "B.Cu") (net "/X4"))
 (segment (start 25.9 13.7) (end 29.7 17.3) (width 0.3) (layer "F.Cu") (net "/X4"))
 (segment (start 29.7 17.3) (end 33.1 21.5) (width 0.3) (layer "B.Cu") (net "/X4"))
 (segment (start 33.1 21.5) (end 33.5 22.24) (width 0.3) (layer "B.Cu") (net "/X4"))
 (segment (start 4 12.08) (end 4.3 11.3) (width 0.3) (layer "B.Cu") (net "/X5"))
 (segment (start 4.3 11.3) (end 5.3 10.3) (width 0.3) (layer "B.Cu") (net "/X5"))
 (segment (start 5.3 10.3) (end 5.3 9.1) (width 0.3) (layer "B.Cu") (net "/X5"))
 (segment (start 5.3 9.1) (end 5.5 8.7) (width 0.3) (layer "B.Cu") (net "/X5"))
 (segment (start 5.5 8.7) (end 5.7 8.5) (width 0.3) (layer "B.Cu") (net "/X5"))
 (segment (start 5.7 8.5) (end 6.1 8.3) (width 0.3) (layer "B.Cu") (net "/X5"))
 (segment (start 6.1 8.3) (end 21.1 8.3) (width 0.3) (layer "B.Cu") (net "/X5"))
 (segment (start 21.1 8.3) (end 23.1 6.3) (width 0.3) (layer "B.Cu") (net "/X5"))
 (segment (start 23.1 6.3) (end 26.1 6.3) (width 0.3) (layer "B.Cu") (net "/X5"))
 (segment (start 26.1 6.3) (end 26.7 5.7) (width 0.3) (layer "B.Cu") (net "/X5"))
 (segment (start 26.7 5.7) (end 34.5 5.7) (width 0.3) (layer "B.Cu") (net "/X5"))
 (segment (start 34.5 5.7) (end 34.7 5.9) (width 0.3) (layer "B.Cu") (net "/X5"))
 (segment (start 34.7 5.9) (end 34.7 7.5) (width 0.3) (layer "B.Cu") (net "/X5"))
 (segment (start 34.7 7.5) (end 35.5 8.3) (width 0.3) (layer "B.Cu") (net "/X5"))
 (segment (start 35.5 8.3) (end 36.5 8.3) (width 0.3) (layer "B.Cu") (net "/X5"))
 (segment (start 36.5 8.3) (end 37.3 9.1) (width 0.3) (layer "B.Cu") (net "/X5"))
 (segment (start 37.3 9.1) (end 37.3 17.9) (width 0.3) (layer "B.Cu") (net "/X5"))
 (segment (start 37.3 17.9) (end 36.3 18.9) (width 0.3) (layer "B.Cu") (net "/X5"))
 (segment (start 36.3 18.9) (end 36.04 19.7) (width 0.3) (layer "B.Cu") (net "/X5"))
 (segment (start 6.54 12.08) (end 7.3 11.7) (width 0.3) (layer "B.Cu") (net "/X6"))
 (segment (start 7.3 11.7) (end 13.1 11.5) (width 0.3) (layer "B.Cu") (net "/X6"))
 (segment (start 13.1 11.5) (end 13.7 12.1) (width 0.3) (layer "B.Cu") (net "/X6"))
 (segment (start 13.7 12.1) (end 16.1 12.1) (width 0.3) (layer "B.Cu") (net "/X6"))
 (segment (start 16.1 12.1) (end 16.9 12.7) (width 0.3) (layer "B.Cu") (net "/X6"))
 (segment (start 16.9 12.7) (end 17.9 15.7) (width 0.3) (layer "F.Cu") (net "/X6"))
 (segment (start 17.9 15.7) (end 19.1 16.9) (width 0.3) (layer "F.Cu") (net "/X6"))
 (segment (start 19.1 16.9) (end 25.3 17.3) (width 0.3) (layer "F.Cu") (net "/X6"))
 (segment (start 25.3 17.3) (end 32.7 19.5) (width 0.3) (layer "F.Cu") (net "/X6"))
 (segment (start 32.7 19.5) (end 33.5 19.7) (width 0.3) (layer "F.Cu") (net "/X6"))
 (segment (start 4 14.62) (end 4.7 15.1) (width 0.3) (layer "F.Cu") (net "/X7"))
 (segment (start 4.7 15.1) (end 5.5 15.9) (width 0.3) (layer "F.Cu") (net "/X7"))
 (segment (start 5.5 15.9) (end 7.1 15.9) (width 0.3) (layer "F.Cu") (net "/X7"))
 (segment (start 7.1 15.9) (end 13.5 17.9) (width 0.3) (layer "F.Cu") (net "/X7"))
 (segment (start 13.5 17.9) (end 16.5 18.1) (width 0.3) (layer "F.Cu") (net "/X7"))
 (segment (start 16.5 18.1) (end 16.7 18.3) (width 0.3) (layer "F.Cu") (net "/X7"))
 (segment (start 16.7 18.3) (end 25.1 18.1) (width 0.3) (layer "F.Cu") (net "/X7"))
 (segment (start 25.1 18.1) (end 25.7 18.7) (width 0.3) (layer "F.Cu") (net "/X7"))
 (segment (start 25.7 18.7) (end 30.9 20.9) (width 0.3) (layer "F.Cu") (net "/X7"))
 (segment (start 30.9 20.9) (end 34.1 20.9) (width 0.3) (layer "F.Cu") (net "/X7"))
 (segment (start 34.1 20.9) (end 34.7 20.3) (width 0.3) (layer "F.Cu") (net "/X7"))
 (segment (start 34.7 20.3) (end 34.7 18.9) (width 0.3) (layer "F.Cu") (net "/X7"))
 (segment (start 34.7 18.9) (end 35.7 17.9) (width 0.3) (layer "F.Cu") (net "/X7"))
 (segment (start 35.7 17.9) (end 36.04 17.16) (width 0.3) (layer "F.Cu") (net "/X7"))
 (segment (start 6.54 14.62) (end 7.3 14.9) (width 0.3) (layer "F.Cu") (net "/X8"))
 (segment (start 7.3 14.9) (end 12.7 16.3) (width 0.3) (layer "F.Cu") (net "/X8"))
 (segment (start 12.7 16.3) (end 15.3 15.5) (width 0.3) (layer "B.Cu") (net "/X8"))
 (segment (start 15.3 15.5) (end 16.5 15.3) (width 0.3) (layer "B.Cu") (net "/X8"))
 (segment (start 16.5 15.3) (end 19.7 13.7) (width 0.3) (layer "B.Cu") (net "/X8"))
 (segment (start 19.7 13.7) (end 20.5 13.7) (width 0.3) (layer "B.Cu") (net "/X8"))
 (segment (start 20.5 13.7) (end 25.9 15.7) (width 0.3) (layer "F.Cu") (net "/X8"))
 (segment (start 25.9 15.7) (end 27.3 15.7) (width 0.3) (layer "B.Cu") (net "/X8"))
 (segment (start 27.3 15.7) (end 28.5 14.5) (width 0.3) (layer "B.Cu") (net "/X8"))
 (segment (start 28.5 14.5) (end 32.9 16.7) (width 0.3) (layer "F.Cu") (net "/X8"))
 (segment (start 32.9 16.7) (end 33.5 17.16) (width 0.3) (layer "F.Cu") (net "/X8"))
 (segment (start 4 17.16) (end 4.3 17.9) (width 0.3) (layer "F.Cu") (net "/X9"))
 (segment (start 4.3 17.9) (end 5.3 19.3) (width 0.3) (layer "F.Cu") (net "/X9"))
 (segment (start 5.3 19.3) (end 5.3 20.1) (width 0.3) (layer "F.Cu") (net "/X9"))
 (segment (start 5.3 20.1) (end 5.5 20.5) (width 0.3) (layer "F.Cu") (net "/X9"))
 (segment (start 5.5 20.5) (end 5.9 20.9) (width 0.3) (layer "F.Cu") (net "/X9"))
 (segment (start 5.9 20.9) (end 7.1 20.9) (width 0.3) (layer "F.Cu") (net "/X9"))
 (segment (start 7.1 20.9) (end 12.5 24.9) (width 0.3) (layer "F.Cu") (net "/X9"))
 (segment (start 12.5 24.9) (end 15.5 24.9) (width 0.3) (layer "F.Cu") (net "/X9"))
 (segment (start 15.5 24.9) (end 22.1 24.3) (width 0.3) (layer "F.Cu") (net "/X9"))
 (segment (start 22.1 24.3) (end 23.7 23.3) (width 0.3) (layer "F.Cu") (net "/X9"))
 (segment (start 23.7 23.3) (end 33.9 23.5) (width 0.3) (layer "F.Cu") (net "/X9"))
 (segment (start 33.9 23.5) (end 34.3 23.3) (width 0.3) (layer "F.Cu") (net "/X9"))
 (segment (start 34.3 23.3) (end 34.7 22.9) (width 0.3) (layer "F.Cu") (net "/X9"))
 (segment (start 34.7 22.9) (end 34.7 21.7) (width 0.3) (layer "F.Cu") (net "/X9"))
 (segment (start 34.7 21.7) (end 35.5 20.9) (width 0.3) (layer "F.Cu") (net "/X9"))
 (segment (start 35.5 20.9) (end 36.7 20.9) (width 0.3) (layer "F.Cu") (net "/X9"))
 (segment (start 36.7 20.9) (end 37.1 20.5) (width 0.3) (layer "F.Cu") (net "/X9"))
 (segment (start 37.1 20.5) (end 37.1 20.3) (width 0.3) (layer "F.Cu") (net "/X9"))
 (segment (start 37.1 20.3) (end 37.3 20.1) (width 0.3) (layer "F.Cu") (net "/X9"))
 (segment (start 37.3 20.1) (end 37.3 16.1) (width 0.3) (layer "F.Cu") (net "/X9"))
 (segment (start 37.3 16.1) (end 36.5 15.3) (width 0.3) (layer "F.Cu") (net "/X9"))
 (segment (start 36.5 15.3) (end 36.04 14.62) (width 0.3) (layer "F.Cu") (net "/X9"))
 (segment (start 4 24.78) (end 4.7 24.7) (width 0.3) (layer "F.Cu") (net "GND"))
 (segment (start 4.7 24.7) (end 5.7 24.7) (width 0.3) (layer "F.Cu") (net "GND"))
 (segment (start 5.7 24.7) (end 6.54 24.78) (width 0.3) (layer "F.Cu") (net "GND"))
 (segment (start 4 24.78) (end 3.3 24.3) (width 0.3) (layer "F.Cu") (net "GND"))
 (segment (start 3.3 24.3) (end 1.1 20.5) (width 0.3) (layer "F.Cu") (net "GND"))
 (segment (start 1.1 20.5) (end 2.7 6.1) (width 0.3) (layer "F.Cu") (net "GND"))
 (segment (start 2.7 6.1) (end 3.1 5.7) (width 0.3) (layer "F.Cu") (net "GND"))
 (segment (start 3.1 5.7) (end 32.7 6.3) (width 0.3) (layer "F.Cu") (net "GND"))
 (segment (start 32.7 6.3) (end 33.5 7) (width 0.3) (layer "F.Cu") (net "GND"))
 (segment (start 33.5 7) (end 34.3 7.1) (width 0.3) (layer "F.Cu") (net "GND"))
 (segment (start 34.3 7.1) (end 35.3 7.1) (width 0.3) (layer "F.Cu") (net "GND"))
 (segment (start 35.3 7.1) (end 36.04 7) (width 0.3) (layer "F.Cu") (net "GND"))
 (via (at 13.7 13.7) (size 0.6) (drill 0.3) (layers "F.Cu" "B.Cu") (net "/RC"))
 (via (at 15.7 13.1) (size 0.6) (drill 0.3) (layers "F.Cu" "B.Cu") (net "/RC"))
 (via (at 16.9 17.3) (size 0.6) (drill 0.3) (layers "F.Cu" "B.Cu") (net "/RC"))
 (via (at 14.3 18.9) (size 0.6) (drill 0.3) (layers "F.Cu" "B.Cu") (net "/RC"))
 (via (at 30.1 12.7) (size 0.6) (drill 0.3) (layers "F.Cu" "B.Cu") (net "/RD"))
 (via (at 16.5 20.7) (size 0.6) (drill 0.3) (layers "F.Cu" "B.Cu") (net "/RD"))
 (via (at 22.3 9.7) (size 0.6) (drill 0.3) (layers "F.Cu" "B.Cu") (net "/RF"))
 (via (at 18.9 15.3) (size 0.6) (drill 0.3) (layers "F.Cu" "B.Cu") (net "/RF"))
 (via (at 14.1 19.9) (size 0.6) (drill 0.3) (layers "F.Cu" "B.Cu") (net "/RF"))
 (via (at 20.7 19.3) (size 0.6) (drill 0.3) (layers "F.Cu" "B.Cu") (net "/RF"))
 (via (at 18.5 20.5) (size 0.6) (drill 0.3) (layers "F.Cu" "B.Cu") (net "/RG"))
 (via (at 21.3 23.1) (size 0.6) (drill 0.3) (layers "F.Cu" "B.Cu") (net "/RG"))
 (via (at 31.9 25.5) (size 0.6) (drill 0.3) (layers "F.Cu" "B.Cu") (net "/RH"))
 (via (at 26.3 24.3) (size 0.6) (drill 0.3) (layers "F.Cu" "B.Cu") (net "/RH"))
 (via (at 21.9 11.9) (size 0.6) (drill 0.3) (layers "F.Cu" "B.Cu") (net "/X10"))
 (via (at 12.7 12.5) (size 0.6) (drill 0.3) (layers "F.Cu" "B.Cu") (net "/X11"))
 (via (at 14.1 11.1) (size 0.6) (drill 0.3) (layers "F.Cu" "B.Cu") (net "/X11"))
 (via (at 22.7 10.9) (size 0.6) (drill 0.3) (layers "F.Cu" "B.Cu") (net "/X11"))
 (via (at 31.9 9.3) (size 0.6) (drill 0.3) (layers "F.Cu" "B.Cu") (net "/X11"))
 (via (at 11.7 22.7) (size 0.6) (drill 0.3) (layers "F.Cu" "B.Cu") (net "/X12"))
 (via (at 25.9 13.7) (size 0.6) (drill 0.3) (layers "F.Cu" "B.Cu") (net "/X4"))
 (via (at 29.7 17.3) (size 0.6) (drill 0.3) (layers "F.Cu" "B.Cu") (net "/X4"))
 (via (at 16.9 12.7) (size 0.6) (drill 0.3) (layers "F.Cu" "B.Cu") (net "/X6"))
 (via (at 12.7 16.3) (size 0.6) (drill 0.3) (layers "F.Cu" "B.Cu") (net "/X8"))
 (via (at 20.5 13.7) (size 0.6) (drill 0.3) (layers "F.Cu" "B.Cu") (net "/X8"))
 (via (at 25.9 15.7) (size 0.6) (drill 0.3) (layers "F.Cu" "B.Cu") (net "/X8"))
 (via (at 28.5 14.5) (size 0.6) (drill 0.3) (layers "F.Cu" "B.Cu") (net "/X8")))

